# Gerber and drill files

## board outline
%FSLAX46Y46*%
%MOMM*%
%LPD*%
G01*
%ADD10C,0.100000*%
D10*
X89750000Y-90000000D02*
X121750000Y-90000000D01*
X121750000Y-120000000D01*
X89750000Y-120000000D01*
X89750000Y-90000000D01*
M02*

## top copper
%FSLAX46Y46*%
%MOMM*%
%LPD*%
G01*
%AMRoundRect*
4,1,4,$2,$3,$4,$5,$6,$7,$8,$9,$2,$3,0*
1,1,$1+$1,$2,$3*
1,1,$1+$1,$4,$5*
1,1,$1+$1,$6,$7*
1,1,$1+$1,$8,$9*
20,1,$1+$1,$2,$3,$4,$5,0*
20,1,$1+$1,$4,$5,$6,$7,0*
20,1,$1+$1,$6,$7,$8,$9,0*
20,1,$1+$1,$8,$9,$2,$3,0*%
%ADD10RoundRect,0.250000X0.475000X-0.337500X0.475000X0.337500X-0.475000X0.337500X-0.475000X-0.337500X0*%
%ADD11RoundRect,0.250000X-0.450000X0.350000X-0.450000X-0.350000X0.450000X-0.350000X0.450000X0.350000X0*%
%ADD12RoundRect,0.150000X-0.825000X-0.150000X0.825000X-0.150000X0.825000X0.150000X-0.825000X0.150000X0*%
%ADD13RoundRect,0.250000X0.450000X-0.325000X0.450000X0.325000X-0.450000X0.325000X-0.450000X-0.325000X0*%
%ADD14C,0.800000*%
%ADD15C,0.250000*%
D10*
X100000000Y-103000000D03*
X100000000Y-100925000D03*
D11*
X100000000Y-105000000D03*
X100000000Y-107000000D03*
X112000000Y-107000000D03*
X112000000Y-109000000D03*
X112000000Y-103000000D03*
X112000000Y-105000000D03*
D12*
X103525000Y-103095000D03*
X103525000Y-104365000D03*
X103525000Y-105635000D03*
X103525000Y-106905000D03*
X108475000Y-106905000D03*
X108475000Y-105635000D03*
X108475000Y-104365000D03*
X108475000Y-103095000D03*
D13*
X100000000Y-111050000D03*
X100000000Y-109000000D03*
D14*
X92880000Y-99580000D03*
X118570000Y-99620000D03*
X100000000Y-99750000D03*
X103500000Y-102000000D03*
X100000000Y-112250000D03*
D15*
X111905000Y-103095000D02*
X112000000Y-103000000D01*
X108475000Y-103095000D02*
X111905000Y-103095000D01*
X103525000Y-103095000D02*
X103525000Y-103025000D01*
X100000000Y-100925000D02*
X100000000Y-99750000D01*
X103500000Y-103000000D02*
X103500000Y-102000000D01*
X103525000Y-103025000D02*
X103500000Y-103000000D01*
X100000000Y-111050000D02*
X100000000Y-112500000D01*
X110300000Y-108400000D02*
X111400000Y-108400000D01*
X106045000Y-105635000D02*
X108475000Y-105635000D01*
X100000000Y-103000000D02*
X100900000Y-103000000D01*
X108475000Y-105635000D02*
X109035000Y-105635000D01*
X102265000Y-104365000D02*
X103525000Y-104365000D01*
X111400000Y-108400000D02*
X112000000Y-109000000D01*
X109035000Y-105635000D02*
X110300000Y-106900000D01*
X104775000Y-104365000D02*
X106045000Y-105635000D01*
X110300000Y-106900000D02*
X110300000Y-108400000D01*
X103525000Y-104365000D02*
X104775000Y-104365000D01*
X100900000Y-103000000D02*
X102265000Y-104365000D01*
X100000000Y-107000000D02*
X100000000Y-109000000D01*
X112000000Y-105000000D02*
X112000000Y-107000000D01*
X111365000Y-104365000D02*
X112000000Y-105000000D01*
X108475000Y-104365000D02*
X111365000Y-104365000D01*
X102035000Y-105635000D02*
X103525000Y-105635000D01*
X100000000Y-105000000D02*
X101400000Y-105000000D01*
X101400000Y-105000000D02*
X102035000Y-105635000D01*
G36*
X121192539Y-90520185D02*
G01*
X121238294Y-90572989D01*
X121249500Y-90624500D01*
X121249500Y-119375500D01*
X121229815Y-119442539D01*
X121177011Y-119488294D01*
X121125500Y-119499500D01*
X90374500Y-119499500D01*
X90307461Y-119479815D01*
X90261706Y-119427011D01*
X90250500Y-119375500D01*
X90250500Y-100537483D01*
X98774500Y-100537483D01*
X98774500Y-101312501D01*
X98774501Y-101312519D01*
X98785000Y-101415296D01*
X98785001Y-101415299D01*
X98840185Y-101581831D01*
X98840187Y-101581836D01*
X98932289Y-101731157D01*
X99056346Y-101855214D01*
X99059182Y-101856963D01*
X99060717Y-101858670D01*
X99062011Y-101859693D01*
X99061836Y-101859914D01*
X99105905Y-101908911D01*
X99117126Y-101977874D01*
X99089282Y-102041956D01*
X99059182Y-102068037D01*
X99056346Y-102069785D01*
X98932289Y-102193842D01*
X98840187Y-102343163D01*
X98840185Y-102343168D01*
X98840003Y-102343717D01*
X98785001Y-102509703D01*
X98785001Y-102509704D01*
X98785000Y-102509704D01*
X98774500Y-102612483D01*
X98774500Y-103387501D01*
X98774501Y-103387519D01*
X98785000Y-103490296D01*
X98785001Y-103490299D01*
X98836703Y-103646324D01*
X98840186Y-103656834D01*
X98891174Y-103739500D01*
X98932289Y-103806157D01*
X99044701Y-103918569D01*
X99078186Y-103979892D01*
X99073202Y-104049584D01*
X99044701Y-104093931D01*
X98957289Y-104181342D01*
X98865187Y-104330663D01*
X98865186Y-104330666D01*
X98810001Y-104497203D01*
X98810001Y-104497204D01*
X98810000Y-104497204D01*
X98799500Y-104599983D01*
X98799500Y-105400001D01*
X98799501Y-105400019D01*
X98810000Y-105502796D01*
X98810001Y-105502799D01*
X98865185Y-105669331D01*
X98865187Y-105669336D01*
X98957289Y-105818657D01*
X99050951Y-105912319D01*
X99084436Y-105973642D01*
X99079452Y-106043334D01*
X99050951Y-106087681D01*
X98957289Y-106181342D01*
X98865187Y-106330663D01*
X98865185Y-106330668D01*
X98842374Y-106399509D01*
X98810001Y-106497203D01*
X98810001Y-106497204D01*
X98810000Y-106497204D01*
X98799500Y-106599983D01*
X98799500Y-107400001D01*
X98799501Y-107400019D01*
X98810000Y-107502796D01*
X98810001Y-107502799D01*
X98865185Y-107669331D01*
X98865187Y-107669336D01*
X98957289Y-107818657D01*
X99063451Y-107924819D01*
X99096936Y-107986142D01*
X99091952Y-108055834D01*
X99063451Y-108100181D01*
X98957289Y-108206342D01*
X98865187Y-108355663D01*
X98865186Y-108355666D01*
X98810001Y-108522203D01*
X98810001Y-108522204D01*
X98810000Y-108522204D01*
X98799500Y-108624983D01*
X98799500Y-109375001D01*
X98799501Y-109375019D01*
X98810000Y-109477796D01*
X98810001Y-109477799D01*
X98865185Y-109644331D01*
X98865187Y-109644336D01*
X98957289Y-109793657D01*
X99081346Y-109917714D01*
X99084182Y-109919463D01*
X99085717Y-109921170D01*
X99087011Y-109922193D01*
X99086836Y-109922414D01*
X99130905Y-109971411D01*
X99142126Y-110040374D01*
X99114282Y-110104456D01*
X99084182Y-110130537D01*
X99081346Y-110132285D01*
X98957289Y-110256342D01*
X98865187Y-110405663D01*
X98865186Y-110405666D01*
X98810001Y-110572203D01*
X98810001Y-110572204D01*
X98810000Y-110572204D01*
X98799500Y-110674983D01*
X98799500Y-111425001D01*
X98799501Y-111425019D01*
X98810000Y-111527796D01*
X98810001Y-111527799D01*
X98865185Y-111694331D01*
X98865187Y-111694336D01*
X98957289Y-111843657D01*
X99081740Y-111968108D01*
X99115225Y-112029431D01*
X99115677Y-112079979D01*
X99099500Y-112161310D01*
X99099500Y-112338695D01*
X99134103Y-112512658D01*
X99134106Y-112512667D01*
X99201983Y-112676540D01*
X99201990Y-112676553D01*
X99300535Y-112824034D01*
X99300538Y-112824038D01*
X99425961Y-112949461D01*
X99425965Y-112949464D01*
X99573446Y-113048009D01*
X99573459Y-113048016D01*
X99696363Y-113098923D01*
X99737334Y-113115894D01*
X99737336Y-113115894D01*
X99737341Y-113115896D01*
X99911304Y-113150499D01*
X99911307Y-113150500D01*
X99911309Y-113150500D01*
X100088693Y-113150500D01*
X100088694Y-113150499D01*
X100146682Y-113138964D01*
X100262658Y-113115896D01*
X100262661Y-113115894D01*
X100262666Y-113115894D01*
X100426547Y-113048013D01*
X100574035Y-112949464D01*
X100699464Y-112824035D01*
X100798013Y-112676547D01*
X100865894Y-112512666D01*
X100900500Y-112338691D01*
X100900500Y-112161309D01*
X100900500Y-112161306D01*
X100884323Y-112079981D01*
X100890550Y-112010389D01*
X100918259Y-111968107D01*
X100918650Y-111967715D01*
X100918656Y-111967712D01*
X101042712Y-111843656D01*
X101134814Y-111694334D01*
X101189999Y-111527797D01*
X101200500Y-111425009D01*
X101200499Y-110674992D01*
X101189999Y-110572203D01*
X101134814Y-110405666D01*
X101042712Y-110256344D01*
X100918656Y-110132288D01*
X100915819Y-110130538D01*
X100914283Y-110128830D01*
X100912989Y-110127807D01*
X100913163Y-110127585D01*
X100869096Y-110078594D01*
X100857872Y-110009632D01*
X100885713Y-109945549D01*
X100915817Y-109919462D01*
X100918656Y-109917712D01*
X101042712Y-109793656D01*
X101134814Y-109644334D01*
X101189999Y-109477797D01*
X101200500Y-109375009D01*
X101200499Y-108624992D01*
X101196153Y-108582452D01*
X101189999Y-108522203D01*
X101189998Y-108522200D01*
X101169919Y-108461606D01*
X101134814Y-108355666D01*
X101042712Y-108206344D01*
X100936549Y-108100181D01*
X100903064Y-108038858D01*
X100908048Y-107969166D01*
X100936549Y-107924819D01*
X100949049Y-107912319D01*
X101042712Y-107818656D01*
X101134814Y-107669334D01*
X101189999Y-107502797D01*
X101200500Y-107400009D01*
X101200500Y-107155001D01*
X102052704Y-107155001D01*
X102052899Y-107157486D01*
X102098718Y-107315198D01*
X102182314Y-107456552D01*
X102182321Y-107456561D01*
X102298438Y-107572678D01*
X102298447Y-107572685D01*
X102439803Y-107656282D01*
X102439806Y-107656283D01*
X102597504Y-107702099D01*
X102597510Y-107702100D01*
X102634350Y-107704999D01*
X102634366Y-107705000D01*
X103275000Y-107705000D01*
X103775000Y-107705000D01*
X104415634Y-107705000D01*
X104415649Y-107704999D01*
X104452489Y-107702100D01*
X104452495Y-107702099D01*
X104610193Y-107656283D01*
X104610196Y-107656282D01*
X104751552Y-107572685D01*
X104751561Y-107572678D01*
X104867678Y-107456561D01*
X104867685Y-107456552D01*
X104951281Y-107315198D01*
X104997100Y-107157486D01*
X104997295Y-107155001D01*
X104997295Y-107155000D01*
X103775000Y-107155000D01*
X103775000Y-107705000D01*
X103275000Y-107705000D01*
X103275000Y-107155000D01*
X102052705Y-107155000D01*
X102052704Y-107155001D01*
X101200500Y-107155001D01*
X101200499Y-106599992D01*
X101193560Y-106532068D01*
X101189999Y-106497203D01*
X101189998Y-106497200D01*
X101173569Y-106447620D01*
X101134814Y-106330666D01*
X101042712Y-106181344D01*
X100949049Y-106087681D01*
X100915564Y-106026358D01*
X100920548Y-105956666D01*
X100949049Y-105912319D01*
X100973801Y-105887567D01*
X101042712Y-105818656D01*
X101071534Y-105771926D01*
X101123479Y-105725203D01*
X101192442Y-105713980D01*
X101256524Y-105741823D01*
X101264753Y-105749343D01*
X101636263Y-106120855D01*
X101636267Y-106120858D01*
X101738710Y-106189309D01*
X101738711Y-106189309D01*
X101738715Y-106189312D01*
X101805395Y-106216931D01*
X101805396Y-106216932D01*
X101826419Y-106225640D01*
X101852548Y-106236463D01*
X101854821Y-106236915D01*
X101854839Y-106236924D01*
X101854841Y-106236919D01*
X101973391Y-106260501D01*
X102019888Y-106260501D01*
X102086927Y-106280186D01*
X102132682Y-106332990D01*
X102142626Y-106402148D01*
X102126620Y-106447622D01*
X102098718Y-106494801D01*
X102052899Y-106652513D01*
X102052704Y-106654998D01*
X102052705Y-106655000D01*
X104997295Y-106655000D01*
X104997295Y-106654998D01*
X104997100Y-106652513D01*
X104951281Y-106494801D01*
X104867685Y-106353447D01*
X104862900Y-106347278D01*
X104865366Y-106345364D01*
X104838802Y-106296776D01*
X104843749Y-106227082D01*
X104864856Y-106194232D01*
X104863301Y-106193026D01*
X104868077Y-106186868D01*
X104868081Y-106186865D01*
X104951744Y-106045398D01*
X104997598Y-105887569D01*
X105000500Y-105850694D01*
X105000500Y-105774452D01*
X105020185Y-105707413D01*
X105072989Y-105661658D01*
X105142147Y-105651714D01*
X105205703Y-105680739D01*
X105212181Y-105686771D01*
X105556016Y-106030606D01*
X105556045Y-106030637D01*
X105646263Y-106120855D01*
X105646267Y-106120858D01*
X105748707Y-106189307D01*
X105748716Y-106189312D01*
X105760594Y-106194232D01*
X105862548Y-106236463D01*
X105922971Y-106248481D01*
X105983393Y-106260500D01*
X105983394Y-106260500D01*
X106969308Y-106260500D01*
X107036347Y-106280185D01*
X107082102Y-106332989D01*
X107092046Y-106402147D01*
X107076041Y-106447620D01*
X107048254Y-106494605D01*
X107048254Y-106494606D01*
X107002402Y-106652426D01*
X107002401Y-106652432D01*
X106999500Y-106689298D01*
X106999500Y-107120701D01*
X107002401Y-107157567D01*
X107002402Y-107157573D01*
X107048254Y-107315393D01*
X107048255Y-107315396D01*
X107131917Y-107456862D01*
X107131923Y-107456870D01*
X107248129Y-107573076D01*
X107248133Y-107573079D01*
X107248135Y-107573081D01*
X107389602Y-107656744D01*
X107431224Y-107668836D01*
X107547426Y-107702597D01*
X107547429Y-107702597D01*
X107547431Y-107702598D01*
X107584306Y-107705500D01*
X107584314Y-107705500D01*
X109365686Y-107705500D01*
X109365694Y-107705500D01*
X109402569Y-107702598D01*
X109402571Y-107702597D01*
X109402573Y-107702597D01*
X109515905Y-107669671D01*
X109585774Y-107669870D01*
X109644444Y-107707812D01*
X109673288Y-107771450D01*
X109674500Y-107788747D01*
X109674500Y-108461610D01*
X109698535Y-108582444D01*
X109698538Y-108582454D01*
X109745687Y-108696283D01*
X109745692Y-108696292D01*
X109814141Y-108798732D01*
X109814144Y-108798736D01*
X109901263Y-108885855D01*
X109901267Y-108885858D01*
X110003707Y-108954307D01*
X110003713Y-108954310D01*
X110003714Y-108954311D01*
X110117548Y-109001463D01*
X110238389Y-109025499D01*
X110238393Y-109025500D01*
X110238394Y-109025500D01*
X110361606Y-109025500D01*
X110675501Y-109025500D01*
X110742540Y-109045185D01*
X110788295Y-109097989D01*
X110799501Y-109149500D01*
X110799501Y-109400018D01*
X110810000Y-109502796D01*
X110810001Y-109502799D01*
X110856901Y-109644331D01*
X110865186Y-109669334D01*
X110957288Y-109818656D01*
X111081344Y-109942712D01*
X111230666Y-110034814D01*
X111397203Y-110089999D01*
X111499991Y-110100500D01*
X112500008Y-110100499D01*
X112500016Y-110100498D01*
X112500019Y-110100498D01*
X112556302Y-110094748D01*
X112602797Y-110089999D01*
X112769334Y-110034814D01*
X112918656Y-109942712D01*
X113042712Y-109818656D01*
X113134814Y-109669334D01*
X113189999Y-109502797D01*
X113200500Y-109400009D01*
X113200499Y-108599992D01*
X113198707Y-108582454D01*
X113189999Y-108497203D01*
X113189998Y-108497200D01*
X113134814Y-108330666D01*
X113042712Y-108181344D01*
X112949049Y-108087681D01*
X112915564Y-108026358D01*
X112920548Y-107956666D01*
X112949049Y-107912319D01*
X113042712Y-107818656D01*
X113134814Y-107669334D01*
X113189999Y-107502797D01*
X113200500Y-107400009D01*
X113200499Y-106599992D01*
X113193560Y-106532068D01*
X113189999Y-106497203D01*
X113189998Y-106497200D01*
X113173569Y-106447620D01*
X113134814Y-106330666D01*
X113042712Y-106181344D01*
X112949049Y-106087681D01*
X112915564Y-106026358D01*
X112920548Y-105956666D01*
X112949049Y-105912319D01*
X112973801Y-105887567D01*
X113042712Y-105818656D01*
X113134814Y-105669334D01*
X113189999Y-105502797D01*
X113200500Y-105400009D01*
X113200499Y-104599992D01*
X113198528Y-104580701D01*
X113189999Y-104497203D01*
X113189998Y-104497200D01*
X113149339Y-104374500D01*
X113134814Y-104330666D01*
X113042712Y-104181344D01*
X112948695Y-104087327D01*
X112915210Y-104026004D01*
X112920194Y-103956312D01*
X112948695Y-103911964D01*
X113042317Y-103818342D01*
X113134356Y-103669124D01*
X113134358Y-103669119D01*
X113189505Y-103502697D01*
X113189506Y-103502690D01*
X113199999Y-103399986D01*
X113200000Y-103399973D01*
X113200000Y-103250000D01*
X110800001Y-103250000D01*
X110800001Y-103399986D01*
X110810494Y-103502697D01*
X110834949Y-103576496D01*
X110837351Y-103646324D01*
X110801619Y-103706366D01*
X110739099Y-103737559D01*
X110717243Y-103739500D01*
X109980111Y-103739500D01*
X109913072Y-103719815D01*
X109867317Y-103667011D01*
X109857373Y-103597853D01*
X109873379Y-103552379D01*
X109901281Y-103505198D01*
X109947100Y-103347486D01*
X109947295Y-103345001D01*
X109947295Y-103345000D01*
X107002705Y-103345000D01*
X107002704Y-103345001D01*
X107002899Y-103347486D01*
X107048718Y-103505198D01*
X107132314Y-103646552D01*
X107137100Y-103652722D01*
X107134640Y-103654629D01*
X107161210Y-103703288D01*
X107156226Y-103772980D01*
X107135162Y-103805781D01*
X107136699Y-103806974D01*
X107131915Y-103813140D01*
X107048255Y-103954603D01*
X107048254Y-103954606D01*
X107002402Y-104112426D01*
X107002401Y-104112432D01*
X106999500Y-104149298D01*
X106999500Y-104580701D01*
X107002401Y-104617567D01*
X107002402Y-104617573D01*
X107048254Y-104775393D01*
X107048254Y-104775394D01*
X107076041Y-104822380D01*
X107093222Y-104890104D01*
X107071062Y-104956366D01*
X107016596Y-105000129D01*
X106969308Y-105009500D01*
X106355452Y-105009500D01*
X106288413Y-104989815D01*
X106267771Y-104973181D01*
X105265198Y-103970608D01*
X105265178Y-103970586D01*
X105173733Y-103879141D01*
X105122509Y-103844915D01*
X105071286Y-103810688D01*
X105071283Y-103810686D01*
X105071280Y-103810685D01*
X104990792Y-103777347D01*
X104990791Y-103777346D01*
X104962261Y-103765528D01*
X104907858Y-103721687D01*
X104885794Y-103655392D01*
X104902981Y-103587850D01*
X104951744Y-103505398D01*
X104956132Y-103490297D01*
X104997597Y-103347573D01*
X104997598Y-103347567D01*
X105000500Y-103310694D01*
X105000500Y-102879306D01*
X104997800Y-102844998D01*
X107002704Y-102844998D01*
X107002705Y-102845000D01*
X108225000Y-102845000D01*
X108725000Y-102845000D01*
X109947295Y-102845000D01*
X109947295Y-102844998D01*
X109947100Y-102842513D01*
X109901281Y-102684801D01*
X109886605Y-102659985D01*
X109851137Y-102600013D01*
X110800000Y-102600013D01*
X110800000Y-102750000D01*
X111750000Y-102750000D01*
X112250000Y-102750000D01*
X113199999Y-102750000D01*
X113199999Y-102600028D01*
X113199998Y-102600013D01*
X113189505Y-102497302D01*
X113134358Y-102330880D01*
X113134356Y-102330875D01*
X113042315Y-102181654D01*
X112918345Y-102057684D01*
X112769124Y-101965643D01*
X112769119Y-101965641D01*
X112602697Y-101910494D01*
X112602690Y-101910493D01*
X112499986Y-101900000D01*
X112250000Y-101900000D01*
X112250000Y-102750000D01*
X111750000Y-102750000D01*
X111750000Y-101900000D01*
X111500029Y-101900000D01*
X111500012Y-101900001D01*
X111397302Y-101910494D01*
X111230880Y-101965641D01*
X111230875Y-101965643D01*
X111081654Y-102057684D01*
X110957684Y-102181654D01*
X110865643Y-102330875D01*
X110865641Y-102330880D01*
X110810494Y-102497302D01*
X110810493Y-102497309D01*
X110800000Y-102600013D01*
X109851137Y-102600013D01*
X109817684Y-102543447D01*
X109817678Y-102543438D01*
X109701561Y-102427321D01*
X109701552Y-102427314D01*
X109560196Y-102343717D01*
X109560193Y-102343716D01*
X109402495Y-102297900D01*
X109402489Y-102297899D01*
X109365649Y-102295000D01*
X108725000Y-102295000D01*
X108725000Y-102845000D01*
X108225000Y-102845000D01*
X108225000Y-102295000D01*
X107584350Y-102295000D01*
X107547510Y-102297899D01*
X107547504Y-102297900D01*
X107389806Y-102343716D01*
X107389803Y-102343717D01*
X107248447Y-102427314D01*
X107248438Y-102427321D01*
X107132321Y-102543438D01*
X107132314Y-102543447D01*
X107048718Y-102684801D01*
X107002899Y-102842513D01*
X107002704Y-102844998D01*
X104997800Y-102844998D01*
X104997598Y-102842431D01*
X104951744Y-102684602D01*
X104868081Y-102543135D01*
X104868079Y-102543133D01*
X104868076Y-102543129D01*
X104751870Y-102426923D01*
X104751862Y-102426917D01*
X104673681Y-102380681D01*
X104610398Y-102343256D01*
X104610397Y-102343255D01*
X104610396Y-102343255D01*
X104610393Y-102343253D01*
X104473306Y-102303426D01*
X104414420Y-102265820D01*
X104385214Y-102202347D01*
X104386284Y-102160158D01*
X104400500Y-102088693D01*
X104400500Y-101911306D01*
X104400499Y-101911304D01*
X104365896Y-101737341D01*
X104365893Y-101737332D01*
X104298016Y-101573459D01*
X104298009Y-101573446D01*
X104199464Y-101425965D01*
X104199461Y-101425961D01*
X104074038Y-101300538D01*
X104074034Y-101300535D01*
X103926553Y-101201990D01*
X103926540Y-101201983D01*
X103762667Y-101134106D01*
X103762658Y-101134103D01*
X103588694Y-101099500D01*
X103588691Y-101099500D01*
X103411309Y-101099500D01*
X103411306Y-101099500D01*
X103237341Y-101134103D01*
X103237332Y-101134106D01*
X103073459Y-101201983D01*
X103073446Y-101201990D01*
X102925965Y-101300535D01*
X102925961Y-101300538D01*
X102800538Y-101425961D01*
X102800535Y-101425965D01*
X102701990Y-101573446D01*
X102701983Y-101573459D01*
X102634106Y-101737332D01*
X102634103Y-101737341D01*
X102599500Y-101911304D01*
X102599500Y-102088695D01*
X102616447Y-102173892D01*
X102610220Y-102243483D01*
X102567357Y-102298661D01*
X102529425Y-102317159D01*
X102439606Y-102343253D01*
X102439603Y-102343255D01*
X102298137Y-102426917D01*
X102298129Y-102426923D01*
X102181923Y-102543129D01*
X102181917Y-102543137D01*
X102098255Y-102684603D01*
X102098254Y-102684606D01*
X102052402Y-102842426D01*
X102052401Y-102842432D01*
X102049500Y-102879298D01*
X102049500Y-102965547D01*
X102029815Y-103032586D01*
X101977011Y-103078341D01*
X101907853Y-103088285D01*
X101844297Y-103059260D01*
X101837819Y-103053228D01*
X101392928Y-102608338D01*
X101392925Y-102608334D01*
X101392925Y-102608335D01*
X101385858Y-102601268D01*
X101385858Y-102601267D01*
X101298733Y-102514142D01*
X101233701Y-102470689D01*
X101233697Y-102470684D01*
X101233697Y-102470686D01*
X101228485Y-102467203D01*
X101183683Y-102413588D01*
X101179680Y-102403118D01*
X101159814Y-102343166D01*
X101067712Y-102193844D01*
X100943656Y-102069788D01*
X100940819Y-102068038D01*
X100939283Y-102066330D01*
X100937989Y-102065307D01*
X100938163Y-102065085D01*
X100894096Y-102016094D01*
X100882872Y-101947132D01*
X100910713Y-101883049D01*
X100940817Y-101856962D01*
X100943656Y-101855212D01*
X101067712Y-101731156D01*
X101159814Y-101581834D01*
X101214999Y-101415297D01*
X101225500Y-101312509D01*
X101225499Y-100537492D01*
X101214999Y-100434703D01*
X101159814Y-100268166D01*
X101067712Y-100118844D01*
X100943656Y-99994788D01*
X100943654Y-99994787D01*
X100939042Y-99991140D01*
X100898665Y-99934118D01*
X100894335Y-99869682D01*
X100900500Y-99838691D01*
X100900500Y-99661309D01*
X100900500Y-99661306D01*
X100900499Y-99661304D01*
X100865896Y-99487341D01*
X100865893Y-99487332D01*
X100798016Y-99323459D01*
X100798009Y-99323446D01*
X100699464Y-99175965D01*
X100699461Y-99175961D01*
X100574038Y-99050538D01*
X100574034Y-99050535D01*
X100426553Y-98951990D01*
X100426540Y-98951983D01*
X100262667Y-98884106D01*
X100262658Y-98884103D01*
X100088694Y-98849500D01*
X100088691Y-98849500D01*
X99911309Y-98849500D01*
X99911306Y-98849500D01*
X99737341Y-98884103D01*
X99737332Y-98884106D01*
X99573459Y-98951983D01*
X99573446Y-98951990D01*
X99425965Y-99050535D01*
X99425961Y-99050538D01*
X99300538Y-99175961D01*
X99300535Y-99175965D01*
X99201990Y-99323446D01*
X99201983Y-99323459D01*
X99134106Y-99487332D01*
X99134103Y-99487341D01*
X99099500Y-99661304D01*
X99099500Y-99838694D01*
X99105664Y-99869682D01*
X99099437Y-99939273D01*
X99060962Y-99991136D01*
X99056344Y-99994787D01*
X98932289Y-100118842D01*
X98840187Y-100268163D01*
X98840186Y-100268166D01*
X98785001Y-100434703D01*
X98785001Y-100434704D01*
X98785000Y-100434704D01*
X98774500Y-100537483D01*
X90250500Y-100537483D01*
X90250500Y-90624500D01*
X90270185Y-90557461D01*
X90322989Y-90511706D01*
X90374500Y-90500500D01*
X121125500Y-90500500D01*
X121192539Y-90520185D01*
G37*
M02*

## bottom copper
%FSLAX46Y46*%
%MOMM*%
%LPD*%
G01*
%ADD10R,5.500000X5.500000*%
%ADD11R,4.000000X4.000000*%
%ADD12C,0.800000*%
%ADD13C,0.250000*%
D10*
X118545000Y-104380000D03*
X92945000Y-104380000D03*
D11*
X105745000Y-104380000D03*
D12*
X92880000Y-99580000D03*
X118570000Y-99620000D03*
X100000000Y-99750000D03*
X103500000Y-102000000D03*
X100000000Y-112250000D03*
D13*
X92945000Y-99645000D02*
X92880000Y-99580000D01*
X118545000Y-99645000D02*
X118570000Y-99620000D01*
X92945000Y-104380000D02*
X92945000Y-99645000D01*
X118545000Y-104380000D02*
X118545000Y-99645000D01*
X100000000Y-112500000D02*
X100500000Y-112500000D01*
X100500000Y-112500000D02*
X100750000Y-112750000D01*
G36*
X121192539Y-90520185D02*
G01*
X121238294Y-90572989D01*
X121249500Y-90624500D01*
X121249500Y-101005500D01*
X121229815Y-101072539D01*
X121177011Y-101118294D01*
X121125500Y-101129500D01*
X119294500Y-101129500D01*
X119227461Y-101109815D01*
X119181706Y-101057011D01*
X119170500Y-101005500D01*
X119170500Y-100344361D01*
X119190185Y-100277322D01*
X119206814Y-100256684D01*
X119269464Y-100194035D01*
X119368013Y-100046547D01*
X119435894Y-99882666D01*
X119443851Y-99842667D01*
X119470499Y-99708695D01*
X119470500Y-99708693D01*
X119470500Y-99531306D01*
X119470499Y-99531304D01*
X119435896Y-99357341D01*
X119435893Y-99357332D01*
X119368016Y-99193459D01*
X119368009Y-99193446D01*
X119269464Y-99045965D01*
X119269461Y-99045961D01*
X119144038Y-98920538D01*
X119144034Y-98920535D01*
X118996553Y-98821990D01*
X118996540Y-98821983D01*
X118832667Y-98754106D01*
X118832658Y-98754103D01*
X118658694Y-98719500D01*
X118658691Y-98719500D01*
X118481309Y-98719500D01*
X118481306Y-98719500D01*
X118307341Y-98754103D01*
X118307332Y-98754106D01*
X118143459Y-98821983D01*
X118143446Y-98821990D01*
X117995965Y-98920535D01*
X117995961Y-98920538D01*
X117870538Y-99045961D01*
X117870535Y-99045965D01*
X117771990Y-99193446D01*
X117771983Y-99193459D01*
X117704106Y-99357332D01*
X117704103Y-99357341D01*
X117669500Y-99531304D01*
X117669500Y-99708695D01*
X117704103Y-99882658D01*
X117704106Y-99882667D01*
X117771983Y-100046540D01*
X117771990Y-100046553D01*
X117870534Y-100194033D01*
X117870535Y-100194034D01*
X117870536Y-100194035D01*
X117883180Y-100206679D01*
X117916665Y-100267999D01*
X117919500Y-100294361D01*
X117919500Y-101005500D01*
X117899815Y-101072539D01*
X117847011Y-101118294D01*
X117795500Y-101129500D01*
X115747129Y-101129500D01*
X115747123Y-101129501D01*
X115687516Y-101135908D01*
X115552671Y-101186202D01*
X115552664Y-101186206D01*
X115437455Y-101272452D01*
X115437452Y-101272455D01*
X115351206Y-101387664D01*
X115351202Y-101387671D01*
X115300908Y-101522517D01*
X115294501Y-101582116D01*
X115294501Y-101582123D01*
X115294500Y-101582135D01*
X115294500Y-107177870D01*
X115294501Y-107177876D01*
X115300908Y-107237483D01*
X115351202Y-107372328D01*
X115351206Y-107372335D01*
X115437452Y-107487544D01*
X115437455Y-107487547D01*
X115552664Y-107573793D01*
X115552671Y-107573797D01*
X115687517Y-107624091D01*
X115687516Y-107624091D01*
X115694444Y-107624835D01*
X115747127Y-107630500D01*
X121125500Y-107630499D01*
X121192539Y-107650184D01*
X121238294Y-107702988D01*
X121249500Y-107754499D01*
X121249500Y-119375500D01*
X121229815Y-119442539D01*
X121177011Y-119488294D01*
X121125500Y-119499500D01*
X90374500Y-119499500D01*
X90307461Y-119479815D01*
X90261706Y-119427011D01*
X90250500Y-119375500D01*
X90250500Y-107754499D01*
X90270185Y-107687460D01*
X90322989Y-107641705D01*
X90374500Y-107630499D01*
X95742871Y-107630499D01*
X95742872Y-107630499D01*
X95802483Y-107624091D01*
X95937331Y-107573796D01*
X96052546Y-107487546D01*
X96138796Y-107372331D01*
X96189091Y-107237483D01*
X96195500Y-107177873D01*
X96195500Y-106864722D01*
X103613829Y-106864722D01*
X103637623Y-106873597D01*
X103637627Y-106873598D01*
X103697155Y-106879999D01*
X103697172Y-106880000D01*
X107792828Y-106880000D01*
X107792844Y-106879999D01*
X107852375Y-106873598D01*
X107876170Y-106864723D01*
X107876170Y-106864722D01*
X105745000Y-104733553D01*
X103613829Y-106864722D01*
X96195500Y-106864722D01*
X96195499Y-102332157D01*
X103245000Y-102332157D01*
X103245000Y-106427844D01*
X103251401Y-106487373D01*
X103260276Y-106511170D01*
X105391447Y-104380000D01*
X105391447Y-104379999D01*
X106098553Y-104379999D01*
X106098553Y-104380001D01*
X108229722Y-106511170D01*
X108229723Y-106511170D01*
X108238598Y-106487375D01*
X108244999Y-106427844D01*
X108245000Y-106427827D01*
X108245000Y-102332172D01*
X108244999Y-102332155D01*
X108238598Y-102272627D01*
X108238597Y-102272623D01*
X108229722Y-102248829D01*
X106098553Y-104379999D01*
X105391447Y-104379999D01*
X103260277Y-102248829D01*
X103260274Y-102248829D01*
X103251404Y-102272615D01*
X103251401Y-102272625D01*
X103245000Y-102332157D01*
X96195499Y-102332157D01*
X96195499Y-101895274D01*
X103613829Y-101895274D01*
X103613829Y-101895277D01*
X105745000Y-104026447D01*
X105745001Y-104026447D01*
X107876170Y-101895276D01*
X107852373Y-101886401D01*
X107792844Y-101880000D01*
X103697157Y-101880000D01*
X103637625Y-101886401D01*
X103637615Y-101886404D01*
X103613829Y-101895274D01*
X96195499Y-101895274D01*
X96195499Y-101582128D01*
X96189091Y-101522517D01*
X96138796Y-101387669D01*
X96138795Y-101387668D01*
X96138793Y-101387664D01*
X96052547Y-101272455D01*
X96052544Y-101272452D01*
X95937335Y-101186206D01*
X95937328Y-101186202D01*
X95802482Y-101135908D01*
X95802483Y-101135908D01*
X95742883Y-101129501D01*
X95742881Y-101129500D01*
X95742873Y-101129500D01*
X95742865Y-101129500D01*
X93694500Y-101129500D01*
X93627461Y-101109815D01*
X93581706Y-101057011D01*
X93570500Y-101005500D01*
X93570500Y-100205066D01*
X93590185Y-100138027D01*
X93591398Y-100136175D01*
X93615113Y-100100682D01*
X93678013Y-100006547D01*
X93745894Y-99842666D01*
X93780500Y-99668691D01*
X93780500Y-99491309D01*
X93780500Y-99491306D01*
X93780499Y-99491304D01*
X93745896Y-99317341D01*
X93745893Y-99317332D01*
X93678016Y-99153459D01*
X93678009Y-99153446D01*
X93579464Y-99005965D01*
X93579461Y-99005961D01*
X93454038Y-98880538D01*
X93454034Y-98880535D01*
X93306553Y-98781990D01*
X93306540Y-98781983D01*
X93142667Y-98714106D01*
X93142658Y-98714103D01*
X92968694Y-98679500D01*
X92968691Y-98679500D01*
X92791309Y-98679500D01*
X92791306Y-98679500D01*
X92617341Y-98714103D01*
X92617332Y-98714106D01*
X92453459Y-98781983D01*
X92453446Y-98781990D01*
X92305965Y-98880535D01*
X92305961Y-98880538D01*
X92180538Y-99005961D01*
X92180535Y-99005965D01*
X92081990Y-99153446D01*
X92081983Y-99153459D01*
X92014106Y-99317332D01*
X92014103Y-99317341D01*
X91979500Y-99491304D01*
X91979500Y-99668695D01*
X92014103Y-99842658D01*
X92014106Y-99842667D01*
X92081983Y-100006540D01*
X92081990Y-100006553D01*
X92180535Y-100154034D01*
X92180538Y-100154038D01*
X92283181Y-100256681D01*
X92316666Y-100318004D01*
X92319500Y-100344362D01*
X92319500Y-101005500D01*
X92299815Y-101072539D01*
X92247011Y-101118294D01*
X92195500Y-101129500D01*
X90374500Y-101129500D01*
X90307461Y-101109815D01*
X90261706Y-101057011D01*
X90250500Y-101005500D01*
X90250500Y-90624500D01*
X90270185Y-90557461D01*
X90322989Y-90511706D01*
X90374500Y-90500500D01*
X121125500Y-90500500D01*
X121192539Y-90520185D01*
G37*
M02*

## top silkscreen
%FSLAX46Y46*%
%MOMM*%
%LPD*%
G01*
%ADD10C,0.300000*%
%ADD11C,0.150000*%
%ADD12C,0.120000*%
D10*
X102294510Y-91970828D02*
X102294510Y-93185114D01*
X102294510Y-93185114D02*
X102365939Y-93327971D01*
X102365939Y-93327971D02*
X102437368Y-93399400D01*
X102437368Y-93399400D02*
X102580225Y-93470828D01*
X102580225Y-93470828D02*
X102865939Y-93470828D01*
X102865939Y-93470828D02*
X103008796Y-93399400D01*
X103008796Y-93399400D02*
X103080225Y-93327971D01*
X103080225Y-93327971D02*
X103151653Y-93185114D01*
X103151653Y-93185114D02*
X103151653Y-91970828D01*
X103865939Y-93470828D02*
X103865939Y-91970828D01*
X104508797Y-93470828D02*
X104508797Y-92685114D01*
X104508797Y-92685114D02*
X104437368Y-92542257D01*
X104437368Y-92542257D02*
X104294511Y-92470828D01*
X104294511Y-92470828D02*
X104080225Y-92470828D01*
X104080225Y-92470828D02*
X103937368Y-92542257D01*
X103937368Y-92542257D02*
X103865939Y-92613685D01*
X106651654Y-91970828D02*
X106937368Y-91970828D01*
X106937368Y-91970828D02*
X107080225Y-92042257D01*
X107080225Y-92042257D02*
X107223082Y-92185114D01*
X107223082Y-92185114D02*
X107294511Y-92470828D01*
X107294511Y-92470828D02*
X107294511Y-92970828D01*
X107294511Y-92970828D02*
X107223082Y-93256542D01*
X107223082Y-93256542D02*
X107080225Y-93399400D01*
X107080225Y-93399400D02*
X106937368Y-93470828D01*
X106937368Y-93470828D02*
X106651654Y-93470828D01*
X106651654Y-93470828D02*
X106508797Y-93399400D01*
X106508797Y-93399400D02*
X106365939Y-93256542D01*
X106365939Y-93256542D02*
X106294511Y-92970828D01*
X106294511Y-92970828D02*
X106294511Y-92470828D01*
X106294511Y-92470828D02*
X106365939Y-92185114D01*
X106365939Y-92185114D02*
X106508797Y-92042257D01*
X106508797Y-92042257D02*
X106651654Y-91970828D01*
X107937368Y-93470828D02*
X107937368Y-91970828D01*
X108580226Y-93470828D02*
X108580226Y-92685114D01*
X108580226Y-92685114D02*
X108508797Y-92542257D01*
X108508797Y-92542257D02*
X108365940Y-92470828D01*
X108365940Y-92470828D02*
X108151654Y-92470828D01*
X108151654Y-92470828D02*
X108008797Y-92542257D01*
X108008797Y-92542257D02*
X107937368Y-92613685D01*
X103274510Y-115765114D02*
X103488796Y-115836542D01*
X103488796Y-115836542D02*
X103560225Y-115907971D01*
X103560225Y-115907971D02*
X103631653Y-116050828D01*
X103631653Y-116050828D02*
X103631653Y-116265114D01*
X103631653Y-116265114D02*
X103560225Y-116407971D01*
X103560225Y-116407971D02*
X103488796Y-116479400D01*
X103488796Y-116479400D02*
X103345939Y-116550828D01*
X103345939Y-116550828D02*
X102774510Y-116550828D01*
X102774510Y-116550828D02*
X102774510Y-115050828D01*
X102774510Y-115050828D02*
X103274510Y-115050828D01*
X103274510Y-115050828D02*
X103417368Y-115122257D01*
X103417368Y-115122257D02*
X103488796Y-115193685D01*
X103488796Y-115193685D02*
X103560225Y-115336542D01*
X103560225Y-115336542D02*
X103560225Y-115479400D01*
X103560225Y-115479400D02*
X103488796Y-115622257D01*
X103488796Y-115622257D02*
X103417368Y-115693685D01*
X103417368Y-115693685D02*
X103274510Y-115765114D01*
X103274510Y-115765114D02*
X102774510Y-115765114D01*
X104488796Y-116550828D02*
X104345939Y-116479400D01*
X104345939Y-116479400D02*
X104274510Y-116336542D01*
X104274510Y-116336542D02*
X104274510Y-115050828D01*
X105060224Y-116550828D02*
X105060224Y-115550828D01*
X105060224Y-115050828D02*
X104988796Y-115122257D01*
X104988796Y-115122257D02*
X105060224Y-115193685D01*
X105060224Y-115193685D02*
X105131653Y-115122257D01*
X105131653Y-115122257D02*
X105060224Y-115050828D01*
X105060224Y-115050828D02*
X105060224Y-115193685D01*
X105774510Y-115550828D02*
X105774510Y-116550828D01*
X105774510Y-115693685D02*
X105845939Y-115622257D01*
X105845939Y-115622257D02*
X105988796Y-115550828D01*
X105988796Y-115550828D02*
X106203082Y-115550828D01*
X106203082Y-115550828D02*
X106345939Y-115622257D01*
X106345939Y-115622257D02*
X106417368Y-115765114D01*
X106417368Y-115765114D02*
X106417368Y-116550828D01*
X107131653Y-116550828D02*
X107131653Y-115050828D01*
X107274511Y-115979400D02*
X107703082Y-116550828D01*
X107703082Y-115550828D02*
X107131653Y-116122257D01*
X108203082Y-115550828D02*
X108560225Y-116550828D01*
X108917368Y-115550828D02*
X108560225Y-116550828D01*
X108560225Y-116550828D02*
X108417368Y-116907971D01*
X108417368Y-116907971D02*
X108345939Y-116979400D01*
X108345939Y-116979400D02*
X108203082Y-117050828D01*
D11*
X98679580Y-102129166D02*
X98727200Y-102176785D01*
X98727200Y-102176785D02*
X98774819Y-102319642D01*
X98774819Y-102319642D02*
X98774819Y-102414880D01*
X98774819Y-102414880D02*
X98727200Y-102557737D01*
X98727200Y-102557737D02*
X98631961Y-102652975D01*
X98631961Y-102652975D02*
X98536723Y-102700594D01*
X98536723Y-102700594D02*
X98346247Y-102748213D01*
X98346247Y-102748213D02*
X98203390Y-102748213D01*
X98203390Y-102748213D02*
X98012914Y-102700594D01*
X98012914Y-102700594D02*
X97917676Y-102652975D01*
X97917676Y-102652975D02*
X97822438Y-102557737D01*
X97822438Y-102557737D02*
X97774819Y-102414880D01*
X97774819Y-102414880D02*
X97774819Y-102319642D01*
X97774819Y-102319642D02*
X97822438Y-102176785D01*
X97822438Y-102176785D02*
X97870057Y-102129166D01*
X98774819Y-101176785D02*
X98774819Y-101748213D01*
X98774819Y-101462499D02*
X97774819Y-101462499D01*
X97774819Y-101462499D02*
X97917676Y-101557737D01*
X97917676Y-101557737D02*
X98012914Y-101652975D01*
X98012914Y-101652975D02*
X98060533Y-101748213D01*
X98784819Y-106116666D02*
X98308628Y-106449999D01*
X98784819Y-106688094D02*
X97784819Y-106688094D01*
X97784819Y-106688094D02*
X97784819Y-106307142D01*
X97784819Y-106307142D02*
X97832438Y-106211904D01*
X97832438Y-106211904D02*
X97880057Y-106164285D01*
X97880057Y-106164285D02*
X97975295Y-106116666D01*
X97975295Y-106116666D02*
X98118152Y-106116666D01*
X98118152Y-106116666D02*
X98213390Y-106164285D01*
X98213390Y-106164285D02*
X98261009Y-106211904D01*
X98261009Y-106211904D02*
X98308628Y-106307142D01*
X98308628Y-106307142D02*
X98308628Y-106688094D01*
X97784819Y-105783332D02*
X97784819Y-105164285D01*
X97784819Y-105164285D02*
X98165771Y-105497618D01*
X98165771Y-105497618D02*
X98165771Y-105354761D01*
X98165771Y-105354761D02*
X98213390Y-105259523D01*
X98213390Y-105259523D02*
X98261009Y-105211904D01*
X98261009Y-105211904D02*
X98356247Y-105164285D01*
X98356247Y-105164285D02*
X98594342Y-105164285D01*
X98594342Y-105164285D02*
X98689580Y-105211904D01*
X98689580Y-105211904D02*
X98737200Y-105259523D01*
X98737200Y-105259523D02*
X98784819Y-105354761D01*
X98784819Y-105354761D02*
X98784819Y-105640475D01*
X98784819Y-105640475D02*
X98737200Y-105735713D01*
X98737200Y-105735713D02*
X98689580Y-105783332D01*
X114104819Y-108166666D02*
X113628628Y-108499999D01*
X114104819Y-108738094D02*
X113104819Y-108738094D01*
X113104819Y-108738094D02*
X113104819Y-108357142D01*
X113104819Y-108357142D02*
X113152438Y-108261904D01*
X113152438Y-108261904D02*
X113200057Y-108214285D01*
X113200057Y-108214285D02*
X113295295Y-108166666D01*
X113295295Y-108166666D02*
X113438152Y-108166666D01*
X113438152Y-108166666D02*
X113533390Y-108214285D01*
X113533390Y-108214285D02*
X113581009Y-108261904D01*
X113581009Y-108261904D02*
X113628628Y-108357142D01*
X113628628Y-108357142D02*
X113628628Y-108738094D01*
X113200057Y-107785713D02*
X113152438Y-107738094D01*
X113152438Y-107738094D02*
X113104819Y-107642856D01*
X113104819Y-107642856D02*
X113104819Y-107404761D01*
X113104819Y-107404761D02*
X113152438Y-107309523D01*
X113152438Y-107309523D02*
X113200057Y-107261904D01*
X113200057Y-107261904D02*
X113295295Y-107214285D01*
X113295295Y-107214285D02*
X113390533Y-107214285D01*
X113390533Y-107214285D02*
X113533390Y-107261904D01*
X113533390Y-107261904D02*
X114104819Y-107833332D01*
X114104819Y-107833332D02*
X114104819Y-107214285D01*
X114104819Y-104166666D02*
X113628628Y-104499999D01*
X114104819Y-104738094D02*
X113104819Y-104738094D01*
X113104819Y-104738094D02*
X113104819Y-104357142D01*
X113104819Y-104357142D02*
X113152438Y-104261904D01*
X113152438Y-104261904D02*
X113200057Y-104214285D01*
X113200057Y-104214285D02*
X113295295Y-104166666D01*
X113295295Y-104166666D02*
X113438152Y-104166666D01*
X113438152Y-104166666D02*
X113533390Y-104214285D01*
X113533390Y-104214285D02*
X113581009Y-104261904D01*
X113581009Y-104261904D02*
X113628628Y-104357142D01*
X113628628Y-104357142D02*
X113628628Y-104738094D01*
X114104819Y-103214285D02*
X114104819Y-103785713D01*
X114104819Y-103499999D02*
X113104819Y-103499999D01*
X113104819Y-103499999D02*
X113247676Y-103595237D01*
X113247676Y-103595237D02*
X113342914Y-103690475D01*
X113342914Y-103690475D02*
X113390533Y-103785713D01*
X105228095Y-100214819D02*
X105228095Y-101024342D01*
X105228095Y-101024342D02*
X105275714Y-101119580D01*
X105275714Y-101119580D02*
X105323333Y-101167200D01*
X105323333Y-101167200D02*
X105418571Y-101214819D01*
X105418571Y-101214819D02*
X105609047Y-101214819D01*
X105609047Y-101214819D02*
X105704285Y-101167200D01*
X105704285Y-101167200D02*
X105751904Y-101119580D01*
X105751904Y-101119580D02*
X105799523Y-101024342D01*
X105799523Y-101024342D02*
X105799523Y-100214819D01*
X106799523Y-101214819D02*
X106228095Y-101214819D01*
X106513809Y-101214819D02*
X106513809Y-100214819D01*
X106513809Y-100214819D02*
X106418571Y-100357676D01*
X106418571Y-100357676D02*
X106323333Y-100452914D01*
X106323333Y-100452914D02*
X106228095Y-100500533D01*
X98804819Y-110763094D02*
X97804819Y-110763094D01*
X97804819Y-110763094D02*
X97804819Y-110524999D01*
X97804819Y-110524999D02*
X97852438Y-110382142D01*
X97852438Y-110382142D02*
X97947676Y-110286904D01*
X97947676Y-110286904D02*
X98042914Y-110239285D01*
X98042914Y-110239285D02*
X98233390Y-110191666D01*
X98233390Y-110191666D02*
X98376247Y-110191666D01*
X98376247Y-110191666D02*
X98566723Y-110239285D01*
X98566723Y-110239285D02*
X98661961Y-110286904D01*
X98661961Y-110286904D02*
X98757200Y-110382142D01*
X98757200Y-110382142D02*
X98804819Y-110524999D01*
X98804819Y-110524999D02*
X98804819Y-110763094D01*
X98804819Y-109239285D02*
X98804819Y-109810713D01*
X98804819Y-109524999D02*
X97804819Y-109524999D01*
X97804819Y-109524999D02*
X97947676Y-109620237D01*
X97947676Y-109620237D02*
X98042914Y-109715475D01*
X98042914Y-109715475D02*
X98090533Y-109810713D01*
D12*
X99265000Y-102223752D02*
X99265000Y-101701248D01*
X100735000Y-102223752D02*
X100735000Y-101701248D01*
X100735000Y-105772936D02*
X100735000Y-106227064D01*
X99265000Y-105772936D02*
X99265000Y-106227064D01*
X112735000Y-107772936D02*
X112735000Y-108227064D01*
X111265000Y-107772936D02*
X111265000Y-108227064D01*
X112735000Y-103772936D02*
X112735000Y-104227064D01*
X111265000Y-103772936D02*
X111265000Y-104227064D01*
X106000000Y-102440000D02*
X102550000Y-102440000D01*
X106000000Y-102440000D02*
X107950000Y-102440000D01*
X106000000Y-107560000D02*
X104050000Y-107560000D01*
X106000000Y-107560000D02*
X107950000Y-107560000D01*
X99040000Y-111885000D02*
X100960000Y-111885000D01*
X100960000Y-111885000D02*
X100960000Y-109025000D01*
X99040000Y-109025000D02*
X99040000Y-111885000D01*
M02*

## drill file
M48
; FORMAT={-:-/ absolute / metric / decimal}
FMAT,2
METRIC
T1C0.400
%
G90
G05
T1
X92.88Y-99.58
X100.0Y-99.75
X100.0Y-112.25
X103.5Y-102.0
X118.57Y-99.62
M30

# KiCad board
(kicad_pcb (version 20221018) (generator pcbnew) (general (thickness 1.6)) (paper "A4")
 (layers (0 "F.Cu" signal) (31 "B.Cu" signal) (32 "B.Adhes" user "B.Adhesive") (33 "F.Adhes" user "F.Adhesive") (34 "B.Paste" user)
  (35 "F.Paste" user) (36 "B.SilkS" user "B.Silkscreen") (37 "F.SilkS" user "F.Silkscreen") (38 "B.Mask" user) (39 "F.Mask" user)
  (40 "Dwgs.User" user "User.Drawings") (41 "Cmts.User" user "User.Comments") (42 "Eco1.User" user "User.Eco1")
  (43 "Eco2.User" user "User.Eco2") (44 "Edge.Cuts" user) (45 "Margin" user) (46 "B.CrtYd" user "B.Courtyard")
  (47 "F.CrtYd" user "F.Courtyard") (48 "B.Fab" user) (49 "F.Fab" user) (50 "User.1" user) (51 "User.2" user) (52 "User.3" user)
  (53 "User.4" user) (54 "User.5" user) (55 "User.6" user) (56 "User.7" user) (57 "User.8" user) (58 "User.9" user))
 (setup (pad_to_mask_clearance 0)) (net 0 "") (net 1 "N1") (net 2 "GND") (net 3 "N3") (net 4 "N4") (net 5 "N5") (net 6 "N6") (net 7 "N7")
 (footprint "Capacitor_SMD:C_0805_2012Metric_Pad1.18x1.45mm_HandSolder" (layer "F.Cu") (at 100 101.9625 90)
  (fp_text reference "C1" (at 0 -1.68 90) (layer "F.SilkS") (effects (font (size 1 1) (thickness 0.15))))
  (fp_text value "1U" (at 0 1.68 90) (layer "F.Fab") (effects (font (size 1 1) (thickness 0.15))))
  (fp_line (start -0.261252 -0.735) (end 0.261252 -0.735) (stroke (width 0.12) (type solid)) (layer "F.SilkS"))
  (fp_line (start -0.261252 0.735) (end 0.261252 0.735) (stroke (width 0.12) (type solid)) (layer "F.SilkS"))
  (pad "1" smd roundrect (at -1.0375 0 90) (size 1.175 1.45) (layers "F.Cu" "F.Paste" "F.Mask") (roundrect_rratio 0.212766) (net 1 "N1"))
  (pad "2" smd roundrect (at 1.0375 0 90) (size 1.175 1.45) (layers "F.Cu" "F.Paste" "F.Mask") (roundrect_rratio 0.212766) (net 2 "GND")))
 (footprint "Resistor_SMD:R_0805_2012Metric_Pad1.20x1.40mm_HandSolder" (layer "F.Cu") (at 100 106 -90)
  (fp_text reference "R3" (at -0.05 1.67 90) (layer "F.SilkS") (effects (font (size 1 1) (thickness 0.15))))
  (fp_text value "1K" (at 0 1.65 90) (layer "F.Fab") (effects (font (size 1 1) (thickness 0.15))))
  (fp_line (start -0.227064 -0.735) (end 0.227064 -0.735) (stroke (width 0.12) (type solid)) (layer "F.SilkS"))
  (fp_line (start -0.227064 0.735) (end 0.227064 0.735) (stroke (width 0.12) (type solid)) (layer "F.SilkS"))
  (pad "1" smd roundrect (at -1 0 270) (size 1.2 1.4) (layers "F.Cu" "F.Paste" "F.Mask") (roundrect_rratio 0.208333) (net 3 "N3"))
  (pad "2" smd roundrect (at 1 0 270) (size 1.2 1.4) (layers "F.Cu" "F.Paste" "F.Mask") (roundrect_rratio 0.208333) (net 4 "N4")))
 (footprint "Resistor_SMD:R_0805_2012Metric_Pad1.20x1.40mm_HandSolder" (layer "F.Cu") (at 112 108 -90)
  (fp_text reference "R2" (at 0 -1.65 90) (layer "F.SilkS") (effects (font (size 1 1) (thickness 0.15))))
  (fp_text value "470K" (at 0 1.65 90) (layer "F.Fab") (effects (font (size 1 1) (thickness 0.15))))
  (fp_line (start -0.227064 -0.735) (end 0.227064 -0.735) (stroke (width 0.12) (type solid)) (layer "F.SilkS"))
  (fp_line (start -0.227064 0.735) (end 0.227064 0.735) (stroke (width 0.12) (type solid)) (layer "F.SilkS"))
  (pad "1" smd roundrect (at -1 0 270) (size 1.2 1.4) (layers "F.Cu" "F.Paste" "F.Mask") (roundrect_rratio 0.208333) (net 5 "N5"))
  (pad "2" smd roundrect (at 1 0 270) (size 1.2 1.4) (layers "F.Cu" "F.Paste" "F.Mask") (roundrect_rratio 0.208333) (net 1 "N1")))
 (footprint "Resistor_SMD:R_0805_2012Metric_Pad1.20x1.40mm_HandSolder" (layer "F.Cu") (at 112 104 -90)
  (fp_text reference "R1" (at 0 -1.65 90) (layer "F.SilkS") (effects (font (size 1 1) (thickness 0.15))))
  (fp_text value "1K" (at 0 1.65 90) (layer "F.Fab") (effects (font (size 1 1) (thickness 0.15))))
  (fp_line (start -0.227064 -0.735) (end 0.227064 -0.735) (stroke (width 0.12) (type solid)) (layer "F.SilkS"))
  (fp_line (start -0.227064 0.735) (end 0.227064 0.735) (stroke (width 0.12) (type solid)) (layer "F.SilkS"))
  (pad "1" smd roundrect (at -1 0 270) (size 1.2 1.4) (layers "F.Cu" "F.Paste" "F.Mask") (roundrect_rratio 0.208333) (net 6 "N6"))
  (pad "2" smd roundrect (at 1 0 270) (size 1.2 1.4) (layers "F.Cu" "F.Paste" "F.Mask") (roundrect_rratio 0.208333) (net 5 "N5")))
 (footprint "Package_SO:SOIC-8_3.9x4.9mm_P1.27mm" (layer "F.Cu") (at 106 105)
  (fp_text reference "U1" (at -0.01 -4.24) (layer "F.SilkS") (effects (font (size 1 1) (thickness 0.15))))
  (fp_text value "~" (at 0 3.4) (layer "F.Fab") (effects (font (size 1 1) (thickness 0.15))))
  (fp_line (start 0 -2.56) (end -3.45 -2.56) (stroke (width 0.12) (type solid)) (layer "F.SilkS"))
  (fp_line (start 0 -2.56) (end 1.95 -2.56) (stroke (width 0.12) (type solid)) (layer "F.SilkS"))
  (fp_line (start 0 2.56) (end -1.95 2.56) (stroke (width 0.12) (type solid)) (layer "F.SilkS"))
  (fp_line (start 0 2.56) (end 1.95 2.56) (stroke (width 0.12) (type solid)) (layer "F.SilkS"))
  (pad "1" smd roundrect (at -2.475 -1.905) (size 1.95 0.6) (layers "F.Cu" "F.Paste" "F.Mask") (roundrect_rratio 0.25) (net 2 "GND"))
  (pad "2" smd roundrect (at -2.475 -0.635) (size 1.95 0.6) (layers "F.Cu" "F.Paste" "F.Mask") (roundrect_rratio 0.25) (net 1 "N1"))
  (pad "3" smd roundrect (at -2.475 0.635) (size 1.95 0.6) (layers "F.Cu" "F.Paste" "F.Mask") (roundrect_rratio 0.25) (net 3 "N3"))
  (pad "4" smd roundrect (at -2.475 1.905) (size 1.95 0.6) (layers "F.Cu" "F.Paste" "F.Mask") (roundrect_rratio 0.25) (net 6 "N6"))
  (pad "5" smd roundrect (at 2.475 1.905) (size 1.95 0.6) (layers "F.Cu" "F.Paste" "F.Mask") (roundrect_rratio 0.25) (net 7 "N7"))
  (pad "6" smd roundrect (at 2.475 0.635) (size 1.95 0.6) (layers "F.Cu" "F.Paste" "F.Mask") (roundrect_rratio 0.25) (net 1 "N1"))
  (pad "7" smd roundrect (at 2.475 -0.635) (size 1.95 0.6) (layers "F.Cu" "F.Paste" "F.Mask") (roundrect_rratio 0.25) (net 5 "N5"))
  (pad "8" smd roundrect (at 2.475 -1.905) (size 1.95 0.6) (layers "F.Cu" "F.Paste" "F.Mask") (roundrect_rratio 0.25) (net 6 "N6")))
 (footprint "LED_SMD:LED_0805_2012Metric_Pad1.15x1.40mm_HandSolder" (layer "F.Cu") (at 100 110.025 90)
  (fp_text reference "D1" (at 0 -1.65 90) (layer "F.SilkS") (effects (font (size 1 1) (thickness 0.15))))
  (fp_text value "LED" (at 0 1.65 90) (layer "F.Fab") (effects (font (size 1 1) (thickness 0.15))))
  (fp_line (start -1.86 -0.96) (end -1.86 0.96) (stroke (width 0.12) (type solid)) (layer "F.SilkS"))
  (fp_line (start -1.86 0.96) (end 1 0.96) (stroke (width 0.12) (type solid)) (layer "F.SilkS"))
  (fp_line (start 1 -0.96) (end -1.86 -0.96) (stroke (width 0.12) (type solid)) (layer "F.SilkS"))
  (pad "1" smd roundrect (at -1.025 0 90) (size 1.15 1.4) (layers "F.Cu" "F.Paste" "F.Mask") (roundrect_rratio 0.217391) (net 2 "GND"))
  (pad "2" smd roundrect (at 1.025 0 90) (size 1.15 1.4) (layers "F.Cu" "F.Paste" "F.Mask") (roundrect_rratio 0.217391) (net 4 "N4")))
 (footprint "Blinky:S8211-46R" (layer "B.Cu") (at 105.745 104.38 180)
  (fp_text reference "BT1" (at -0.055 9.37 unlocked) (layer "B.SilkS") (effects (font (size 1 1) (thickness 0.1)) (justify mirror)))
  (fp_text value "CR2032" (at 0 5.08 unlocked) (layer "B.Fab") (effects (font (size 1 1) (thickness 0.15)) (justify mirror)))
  (pad "1" smd rect (at -12.8 0 180) (size 5.5 5.5) (layers "B.Cu" "B.Paste" "B.Mask") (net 6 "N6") (thermal_bridge_angle 45))
  (pad "1" smd rect (at 12.8 0 180) (size 5.5 5.5) (layers "B.Cu" "B.Paste" "B.Mask") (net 6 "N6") (thermal_bridge_angle 45))
  (pad "2" smd rect (at 0 0 180) (size 4 4) (layers "B.Cu" "B.Paste" "B.Mask") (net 2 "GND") (thermal_bridge_angle 45)))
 (gr_rect (start 89.75 90) (end 121.75 120) (stroke (width 0.1) (type default)) (fill none) (layer "Edge.Cuts"))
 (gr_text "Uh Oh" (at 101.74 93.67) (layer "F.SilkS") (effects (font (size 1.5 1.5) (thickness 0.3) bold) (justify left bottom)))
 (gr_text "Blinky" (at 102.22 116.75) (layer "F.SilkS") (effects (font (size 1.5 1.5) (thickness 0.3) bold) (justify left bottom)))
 (segment (start 111.905 103.095) (end 112 103) (width 0.25) (layer "F.Cu") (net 6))
 (segment (start 108.475 103.095) (end 111.905 103.095) (width 0.25) (layer "F.Cu") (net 6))
 (via (at 92.88 99.58) (size 0.8) (drill 0.4) (layers "F.Cu" "B.Cu") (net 6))
 (via (at 118.57 99.62) (size 0.8) (drill 0.4) (layers "F.Cu" "B.Cu") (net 6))
 (segment (start 92.945 99.645) (end 92.88 99.58) (width 0.25) (layer "B.Cu") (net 6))
 (segment (start 118.545 99.645) (end 118.57 99.62) (width 0.25) (layer "B.Cu") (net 6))
 (segment (start 92.945 104.38) (end 92.945 99.645) (width 0.25) (layer "B.Cu") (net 6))
 (segment (start 118.545 104.38) (end 118.545 99.645) (width 0.25) (layer "B.Cu") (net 6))
 (segment (start 103.525 103.095) (end 103.525 103.025) (width 0.25) (layer "F.Cu") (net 2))
 (segment (start 100 100.925) (end 100 99.75) (width 0.25) (layer "F.Cu") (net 2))
 (segment (start 103.5 103) (end 103.5 102) (width 0.25) (layer "F.Cu") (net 2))
 (segment (start 103.525 103.025) (end 103.5 103) (width 0.25) (layer "F.Cu") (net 2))
 (segment (start 100 111.05) (end 100 112.5) (width 0.25) (layer "F.Cu") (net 2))
 (via (at 100 99.75) (size 0.8) (drill 0.4) (layers "F.Cu" "B.Cu") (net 2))
 (via (at 103.5 102) (size 0.8) (drill 0.4) (layers "F.Cu" "B.Cu") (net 2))
 (via (at 100 112.25) (size 0.8) (drill 0.4) (layers "F.Cu" "B.Cu") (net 2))
 (segment (start 100 112.5) (end 100.5 112.5) (width 0.25) (layer "B.Cu") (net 2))
 (segment (start 100.5 112.5) (end 100.75 112.75) (width 0.25) (layer "B.Cu") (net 2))
 (segment (start 110.3 108.4) (end 111.4 108.4) (width 0.25) (layer "F.Cu") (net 1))
 (segment (start 106.045 105.635) (end 108.475 105.635) (width 0.25) (layer "F.Cu") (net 1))
 (segment (start 100 103) (end 100.9 103) (width 0.25) (layer "F.Cu") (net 1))
 (segment (start 108.475 105.635) (end 109.035 105.635) (width 0.25) (layer "F.Cu") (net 1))
 (segment (start 102.265 104.365) (end 103.525 104.365) (width 0.25) (layer "F.Cu") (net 1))
 (segment (start 111.4 108.4) (end 112 109) (width 0.25) (layer "F.Cu") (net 1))
 (segment (start 109.035 105.635) (end 110.3 106.9) (width 0.25) (layer "F.Cu") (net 1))
 (segment (start 104.775 104.365) (end 106.045 105.635) (width 0.25) (layer "F.Cu") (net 1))
 (segment (start 110.3 106.9) (end 110.3 108.4) (width 0.25) (layer "F.Cu") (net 1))
 (segment (start 103.525 104.365) (end 104.775 104.365) (width 0.25) (layer "F.Cu") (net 1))
 (segment (start 100.9 103) (end 102.265 104.365) (width 0.25) (layer "F.Cu") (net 1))
 (segment (start 100 107) (end 100 109) (width 0.25) (layer "F.Cu") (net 4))
 (segment (start 112 105) (end 112 107) (width 0.25) (layer "F.Cu") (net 5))
 (segment (start 111.365 104.365) (end 112 105) (width 0.25) (layer "F.Cu") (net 5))
 (segment (start 108.475 104.365) (end 111.365 104.365) (width 0.25) (layer "F.Cu") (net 5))
 (segment (start 102.035 105.635) (end 103.525 105.635) (width 0.25) (layer "F.Cu") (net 3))
 (segment (start 100 105) (end 101.4 105) (width 0.25) (layer "F.Cu") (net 3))
 (segment (start 101.4 105) (end 102.035 105.635) (width 0.25) (layer "F.Cu") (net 3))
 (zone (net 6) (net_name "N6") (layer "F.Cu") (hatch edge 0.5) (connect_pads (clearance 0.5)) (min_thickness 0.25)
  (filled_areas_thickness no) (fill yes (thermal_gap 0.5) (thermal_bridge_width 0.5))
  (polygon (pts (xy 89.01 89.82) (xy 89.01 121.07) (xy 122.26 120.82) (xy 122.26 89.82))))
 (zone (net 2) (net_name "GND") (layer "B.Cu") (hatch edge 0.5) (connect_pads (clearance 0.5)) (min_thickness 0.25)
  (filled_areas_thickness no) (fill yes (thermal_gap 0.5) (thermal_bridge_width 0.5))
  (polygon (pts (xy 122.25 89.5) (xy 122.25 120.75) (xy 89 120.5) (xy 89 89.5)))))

